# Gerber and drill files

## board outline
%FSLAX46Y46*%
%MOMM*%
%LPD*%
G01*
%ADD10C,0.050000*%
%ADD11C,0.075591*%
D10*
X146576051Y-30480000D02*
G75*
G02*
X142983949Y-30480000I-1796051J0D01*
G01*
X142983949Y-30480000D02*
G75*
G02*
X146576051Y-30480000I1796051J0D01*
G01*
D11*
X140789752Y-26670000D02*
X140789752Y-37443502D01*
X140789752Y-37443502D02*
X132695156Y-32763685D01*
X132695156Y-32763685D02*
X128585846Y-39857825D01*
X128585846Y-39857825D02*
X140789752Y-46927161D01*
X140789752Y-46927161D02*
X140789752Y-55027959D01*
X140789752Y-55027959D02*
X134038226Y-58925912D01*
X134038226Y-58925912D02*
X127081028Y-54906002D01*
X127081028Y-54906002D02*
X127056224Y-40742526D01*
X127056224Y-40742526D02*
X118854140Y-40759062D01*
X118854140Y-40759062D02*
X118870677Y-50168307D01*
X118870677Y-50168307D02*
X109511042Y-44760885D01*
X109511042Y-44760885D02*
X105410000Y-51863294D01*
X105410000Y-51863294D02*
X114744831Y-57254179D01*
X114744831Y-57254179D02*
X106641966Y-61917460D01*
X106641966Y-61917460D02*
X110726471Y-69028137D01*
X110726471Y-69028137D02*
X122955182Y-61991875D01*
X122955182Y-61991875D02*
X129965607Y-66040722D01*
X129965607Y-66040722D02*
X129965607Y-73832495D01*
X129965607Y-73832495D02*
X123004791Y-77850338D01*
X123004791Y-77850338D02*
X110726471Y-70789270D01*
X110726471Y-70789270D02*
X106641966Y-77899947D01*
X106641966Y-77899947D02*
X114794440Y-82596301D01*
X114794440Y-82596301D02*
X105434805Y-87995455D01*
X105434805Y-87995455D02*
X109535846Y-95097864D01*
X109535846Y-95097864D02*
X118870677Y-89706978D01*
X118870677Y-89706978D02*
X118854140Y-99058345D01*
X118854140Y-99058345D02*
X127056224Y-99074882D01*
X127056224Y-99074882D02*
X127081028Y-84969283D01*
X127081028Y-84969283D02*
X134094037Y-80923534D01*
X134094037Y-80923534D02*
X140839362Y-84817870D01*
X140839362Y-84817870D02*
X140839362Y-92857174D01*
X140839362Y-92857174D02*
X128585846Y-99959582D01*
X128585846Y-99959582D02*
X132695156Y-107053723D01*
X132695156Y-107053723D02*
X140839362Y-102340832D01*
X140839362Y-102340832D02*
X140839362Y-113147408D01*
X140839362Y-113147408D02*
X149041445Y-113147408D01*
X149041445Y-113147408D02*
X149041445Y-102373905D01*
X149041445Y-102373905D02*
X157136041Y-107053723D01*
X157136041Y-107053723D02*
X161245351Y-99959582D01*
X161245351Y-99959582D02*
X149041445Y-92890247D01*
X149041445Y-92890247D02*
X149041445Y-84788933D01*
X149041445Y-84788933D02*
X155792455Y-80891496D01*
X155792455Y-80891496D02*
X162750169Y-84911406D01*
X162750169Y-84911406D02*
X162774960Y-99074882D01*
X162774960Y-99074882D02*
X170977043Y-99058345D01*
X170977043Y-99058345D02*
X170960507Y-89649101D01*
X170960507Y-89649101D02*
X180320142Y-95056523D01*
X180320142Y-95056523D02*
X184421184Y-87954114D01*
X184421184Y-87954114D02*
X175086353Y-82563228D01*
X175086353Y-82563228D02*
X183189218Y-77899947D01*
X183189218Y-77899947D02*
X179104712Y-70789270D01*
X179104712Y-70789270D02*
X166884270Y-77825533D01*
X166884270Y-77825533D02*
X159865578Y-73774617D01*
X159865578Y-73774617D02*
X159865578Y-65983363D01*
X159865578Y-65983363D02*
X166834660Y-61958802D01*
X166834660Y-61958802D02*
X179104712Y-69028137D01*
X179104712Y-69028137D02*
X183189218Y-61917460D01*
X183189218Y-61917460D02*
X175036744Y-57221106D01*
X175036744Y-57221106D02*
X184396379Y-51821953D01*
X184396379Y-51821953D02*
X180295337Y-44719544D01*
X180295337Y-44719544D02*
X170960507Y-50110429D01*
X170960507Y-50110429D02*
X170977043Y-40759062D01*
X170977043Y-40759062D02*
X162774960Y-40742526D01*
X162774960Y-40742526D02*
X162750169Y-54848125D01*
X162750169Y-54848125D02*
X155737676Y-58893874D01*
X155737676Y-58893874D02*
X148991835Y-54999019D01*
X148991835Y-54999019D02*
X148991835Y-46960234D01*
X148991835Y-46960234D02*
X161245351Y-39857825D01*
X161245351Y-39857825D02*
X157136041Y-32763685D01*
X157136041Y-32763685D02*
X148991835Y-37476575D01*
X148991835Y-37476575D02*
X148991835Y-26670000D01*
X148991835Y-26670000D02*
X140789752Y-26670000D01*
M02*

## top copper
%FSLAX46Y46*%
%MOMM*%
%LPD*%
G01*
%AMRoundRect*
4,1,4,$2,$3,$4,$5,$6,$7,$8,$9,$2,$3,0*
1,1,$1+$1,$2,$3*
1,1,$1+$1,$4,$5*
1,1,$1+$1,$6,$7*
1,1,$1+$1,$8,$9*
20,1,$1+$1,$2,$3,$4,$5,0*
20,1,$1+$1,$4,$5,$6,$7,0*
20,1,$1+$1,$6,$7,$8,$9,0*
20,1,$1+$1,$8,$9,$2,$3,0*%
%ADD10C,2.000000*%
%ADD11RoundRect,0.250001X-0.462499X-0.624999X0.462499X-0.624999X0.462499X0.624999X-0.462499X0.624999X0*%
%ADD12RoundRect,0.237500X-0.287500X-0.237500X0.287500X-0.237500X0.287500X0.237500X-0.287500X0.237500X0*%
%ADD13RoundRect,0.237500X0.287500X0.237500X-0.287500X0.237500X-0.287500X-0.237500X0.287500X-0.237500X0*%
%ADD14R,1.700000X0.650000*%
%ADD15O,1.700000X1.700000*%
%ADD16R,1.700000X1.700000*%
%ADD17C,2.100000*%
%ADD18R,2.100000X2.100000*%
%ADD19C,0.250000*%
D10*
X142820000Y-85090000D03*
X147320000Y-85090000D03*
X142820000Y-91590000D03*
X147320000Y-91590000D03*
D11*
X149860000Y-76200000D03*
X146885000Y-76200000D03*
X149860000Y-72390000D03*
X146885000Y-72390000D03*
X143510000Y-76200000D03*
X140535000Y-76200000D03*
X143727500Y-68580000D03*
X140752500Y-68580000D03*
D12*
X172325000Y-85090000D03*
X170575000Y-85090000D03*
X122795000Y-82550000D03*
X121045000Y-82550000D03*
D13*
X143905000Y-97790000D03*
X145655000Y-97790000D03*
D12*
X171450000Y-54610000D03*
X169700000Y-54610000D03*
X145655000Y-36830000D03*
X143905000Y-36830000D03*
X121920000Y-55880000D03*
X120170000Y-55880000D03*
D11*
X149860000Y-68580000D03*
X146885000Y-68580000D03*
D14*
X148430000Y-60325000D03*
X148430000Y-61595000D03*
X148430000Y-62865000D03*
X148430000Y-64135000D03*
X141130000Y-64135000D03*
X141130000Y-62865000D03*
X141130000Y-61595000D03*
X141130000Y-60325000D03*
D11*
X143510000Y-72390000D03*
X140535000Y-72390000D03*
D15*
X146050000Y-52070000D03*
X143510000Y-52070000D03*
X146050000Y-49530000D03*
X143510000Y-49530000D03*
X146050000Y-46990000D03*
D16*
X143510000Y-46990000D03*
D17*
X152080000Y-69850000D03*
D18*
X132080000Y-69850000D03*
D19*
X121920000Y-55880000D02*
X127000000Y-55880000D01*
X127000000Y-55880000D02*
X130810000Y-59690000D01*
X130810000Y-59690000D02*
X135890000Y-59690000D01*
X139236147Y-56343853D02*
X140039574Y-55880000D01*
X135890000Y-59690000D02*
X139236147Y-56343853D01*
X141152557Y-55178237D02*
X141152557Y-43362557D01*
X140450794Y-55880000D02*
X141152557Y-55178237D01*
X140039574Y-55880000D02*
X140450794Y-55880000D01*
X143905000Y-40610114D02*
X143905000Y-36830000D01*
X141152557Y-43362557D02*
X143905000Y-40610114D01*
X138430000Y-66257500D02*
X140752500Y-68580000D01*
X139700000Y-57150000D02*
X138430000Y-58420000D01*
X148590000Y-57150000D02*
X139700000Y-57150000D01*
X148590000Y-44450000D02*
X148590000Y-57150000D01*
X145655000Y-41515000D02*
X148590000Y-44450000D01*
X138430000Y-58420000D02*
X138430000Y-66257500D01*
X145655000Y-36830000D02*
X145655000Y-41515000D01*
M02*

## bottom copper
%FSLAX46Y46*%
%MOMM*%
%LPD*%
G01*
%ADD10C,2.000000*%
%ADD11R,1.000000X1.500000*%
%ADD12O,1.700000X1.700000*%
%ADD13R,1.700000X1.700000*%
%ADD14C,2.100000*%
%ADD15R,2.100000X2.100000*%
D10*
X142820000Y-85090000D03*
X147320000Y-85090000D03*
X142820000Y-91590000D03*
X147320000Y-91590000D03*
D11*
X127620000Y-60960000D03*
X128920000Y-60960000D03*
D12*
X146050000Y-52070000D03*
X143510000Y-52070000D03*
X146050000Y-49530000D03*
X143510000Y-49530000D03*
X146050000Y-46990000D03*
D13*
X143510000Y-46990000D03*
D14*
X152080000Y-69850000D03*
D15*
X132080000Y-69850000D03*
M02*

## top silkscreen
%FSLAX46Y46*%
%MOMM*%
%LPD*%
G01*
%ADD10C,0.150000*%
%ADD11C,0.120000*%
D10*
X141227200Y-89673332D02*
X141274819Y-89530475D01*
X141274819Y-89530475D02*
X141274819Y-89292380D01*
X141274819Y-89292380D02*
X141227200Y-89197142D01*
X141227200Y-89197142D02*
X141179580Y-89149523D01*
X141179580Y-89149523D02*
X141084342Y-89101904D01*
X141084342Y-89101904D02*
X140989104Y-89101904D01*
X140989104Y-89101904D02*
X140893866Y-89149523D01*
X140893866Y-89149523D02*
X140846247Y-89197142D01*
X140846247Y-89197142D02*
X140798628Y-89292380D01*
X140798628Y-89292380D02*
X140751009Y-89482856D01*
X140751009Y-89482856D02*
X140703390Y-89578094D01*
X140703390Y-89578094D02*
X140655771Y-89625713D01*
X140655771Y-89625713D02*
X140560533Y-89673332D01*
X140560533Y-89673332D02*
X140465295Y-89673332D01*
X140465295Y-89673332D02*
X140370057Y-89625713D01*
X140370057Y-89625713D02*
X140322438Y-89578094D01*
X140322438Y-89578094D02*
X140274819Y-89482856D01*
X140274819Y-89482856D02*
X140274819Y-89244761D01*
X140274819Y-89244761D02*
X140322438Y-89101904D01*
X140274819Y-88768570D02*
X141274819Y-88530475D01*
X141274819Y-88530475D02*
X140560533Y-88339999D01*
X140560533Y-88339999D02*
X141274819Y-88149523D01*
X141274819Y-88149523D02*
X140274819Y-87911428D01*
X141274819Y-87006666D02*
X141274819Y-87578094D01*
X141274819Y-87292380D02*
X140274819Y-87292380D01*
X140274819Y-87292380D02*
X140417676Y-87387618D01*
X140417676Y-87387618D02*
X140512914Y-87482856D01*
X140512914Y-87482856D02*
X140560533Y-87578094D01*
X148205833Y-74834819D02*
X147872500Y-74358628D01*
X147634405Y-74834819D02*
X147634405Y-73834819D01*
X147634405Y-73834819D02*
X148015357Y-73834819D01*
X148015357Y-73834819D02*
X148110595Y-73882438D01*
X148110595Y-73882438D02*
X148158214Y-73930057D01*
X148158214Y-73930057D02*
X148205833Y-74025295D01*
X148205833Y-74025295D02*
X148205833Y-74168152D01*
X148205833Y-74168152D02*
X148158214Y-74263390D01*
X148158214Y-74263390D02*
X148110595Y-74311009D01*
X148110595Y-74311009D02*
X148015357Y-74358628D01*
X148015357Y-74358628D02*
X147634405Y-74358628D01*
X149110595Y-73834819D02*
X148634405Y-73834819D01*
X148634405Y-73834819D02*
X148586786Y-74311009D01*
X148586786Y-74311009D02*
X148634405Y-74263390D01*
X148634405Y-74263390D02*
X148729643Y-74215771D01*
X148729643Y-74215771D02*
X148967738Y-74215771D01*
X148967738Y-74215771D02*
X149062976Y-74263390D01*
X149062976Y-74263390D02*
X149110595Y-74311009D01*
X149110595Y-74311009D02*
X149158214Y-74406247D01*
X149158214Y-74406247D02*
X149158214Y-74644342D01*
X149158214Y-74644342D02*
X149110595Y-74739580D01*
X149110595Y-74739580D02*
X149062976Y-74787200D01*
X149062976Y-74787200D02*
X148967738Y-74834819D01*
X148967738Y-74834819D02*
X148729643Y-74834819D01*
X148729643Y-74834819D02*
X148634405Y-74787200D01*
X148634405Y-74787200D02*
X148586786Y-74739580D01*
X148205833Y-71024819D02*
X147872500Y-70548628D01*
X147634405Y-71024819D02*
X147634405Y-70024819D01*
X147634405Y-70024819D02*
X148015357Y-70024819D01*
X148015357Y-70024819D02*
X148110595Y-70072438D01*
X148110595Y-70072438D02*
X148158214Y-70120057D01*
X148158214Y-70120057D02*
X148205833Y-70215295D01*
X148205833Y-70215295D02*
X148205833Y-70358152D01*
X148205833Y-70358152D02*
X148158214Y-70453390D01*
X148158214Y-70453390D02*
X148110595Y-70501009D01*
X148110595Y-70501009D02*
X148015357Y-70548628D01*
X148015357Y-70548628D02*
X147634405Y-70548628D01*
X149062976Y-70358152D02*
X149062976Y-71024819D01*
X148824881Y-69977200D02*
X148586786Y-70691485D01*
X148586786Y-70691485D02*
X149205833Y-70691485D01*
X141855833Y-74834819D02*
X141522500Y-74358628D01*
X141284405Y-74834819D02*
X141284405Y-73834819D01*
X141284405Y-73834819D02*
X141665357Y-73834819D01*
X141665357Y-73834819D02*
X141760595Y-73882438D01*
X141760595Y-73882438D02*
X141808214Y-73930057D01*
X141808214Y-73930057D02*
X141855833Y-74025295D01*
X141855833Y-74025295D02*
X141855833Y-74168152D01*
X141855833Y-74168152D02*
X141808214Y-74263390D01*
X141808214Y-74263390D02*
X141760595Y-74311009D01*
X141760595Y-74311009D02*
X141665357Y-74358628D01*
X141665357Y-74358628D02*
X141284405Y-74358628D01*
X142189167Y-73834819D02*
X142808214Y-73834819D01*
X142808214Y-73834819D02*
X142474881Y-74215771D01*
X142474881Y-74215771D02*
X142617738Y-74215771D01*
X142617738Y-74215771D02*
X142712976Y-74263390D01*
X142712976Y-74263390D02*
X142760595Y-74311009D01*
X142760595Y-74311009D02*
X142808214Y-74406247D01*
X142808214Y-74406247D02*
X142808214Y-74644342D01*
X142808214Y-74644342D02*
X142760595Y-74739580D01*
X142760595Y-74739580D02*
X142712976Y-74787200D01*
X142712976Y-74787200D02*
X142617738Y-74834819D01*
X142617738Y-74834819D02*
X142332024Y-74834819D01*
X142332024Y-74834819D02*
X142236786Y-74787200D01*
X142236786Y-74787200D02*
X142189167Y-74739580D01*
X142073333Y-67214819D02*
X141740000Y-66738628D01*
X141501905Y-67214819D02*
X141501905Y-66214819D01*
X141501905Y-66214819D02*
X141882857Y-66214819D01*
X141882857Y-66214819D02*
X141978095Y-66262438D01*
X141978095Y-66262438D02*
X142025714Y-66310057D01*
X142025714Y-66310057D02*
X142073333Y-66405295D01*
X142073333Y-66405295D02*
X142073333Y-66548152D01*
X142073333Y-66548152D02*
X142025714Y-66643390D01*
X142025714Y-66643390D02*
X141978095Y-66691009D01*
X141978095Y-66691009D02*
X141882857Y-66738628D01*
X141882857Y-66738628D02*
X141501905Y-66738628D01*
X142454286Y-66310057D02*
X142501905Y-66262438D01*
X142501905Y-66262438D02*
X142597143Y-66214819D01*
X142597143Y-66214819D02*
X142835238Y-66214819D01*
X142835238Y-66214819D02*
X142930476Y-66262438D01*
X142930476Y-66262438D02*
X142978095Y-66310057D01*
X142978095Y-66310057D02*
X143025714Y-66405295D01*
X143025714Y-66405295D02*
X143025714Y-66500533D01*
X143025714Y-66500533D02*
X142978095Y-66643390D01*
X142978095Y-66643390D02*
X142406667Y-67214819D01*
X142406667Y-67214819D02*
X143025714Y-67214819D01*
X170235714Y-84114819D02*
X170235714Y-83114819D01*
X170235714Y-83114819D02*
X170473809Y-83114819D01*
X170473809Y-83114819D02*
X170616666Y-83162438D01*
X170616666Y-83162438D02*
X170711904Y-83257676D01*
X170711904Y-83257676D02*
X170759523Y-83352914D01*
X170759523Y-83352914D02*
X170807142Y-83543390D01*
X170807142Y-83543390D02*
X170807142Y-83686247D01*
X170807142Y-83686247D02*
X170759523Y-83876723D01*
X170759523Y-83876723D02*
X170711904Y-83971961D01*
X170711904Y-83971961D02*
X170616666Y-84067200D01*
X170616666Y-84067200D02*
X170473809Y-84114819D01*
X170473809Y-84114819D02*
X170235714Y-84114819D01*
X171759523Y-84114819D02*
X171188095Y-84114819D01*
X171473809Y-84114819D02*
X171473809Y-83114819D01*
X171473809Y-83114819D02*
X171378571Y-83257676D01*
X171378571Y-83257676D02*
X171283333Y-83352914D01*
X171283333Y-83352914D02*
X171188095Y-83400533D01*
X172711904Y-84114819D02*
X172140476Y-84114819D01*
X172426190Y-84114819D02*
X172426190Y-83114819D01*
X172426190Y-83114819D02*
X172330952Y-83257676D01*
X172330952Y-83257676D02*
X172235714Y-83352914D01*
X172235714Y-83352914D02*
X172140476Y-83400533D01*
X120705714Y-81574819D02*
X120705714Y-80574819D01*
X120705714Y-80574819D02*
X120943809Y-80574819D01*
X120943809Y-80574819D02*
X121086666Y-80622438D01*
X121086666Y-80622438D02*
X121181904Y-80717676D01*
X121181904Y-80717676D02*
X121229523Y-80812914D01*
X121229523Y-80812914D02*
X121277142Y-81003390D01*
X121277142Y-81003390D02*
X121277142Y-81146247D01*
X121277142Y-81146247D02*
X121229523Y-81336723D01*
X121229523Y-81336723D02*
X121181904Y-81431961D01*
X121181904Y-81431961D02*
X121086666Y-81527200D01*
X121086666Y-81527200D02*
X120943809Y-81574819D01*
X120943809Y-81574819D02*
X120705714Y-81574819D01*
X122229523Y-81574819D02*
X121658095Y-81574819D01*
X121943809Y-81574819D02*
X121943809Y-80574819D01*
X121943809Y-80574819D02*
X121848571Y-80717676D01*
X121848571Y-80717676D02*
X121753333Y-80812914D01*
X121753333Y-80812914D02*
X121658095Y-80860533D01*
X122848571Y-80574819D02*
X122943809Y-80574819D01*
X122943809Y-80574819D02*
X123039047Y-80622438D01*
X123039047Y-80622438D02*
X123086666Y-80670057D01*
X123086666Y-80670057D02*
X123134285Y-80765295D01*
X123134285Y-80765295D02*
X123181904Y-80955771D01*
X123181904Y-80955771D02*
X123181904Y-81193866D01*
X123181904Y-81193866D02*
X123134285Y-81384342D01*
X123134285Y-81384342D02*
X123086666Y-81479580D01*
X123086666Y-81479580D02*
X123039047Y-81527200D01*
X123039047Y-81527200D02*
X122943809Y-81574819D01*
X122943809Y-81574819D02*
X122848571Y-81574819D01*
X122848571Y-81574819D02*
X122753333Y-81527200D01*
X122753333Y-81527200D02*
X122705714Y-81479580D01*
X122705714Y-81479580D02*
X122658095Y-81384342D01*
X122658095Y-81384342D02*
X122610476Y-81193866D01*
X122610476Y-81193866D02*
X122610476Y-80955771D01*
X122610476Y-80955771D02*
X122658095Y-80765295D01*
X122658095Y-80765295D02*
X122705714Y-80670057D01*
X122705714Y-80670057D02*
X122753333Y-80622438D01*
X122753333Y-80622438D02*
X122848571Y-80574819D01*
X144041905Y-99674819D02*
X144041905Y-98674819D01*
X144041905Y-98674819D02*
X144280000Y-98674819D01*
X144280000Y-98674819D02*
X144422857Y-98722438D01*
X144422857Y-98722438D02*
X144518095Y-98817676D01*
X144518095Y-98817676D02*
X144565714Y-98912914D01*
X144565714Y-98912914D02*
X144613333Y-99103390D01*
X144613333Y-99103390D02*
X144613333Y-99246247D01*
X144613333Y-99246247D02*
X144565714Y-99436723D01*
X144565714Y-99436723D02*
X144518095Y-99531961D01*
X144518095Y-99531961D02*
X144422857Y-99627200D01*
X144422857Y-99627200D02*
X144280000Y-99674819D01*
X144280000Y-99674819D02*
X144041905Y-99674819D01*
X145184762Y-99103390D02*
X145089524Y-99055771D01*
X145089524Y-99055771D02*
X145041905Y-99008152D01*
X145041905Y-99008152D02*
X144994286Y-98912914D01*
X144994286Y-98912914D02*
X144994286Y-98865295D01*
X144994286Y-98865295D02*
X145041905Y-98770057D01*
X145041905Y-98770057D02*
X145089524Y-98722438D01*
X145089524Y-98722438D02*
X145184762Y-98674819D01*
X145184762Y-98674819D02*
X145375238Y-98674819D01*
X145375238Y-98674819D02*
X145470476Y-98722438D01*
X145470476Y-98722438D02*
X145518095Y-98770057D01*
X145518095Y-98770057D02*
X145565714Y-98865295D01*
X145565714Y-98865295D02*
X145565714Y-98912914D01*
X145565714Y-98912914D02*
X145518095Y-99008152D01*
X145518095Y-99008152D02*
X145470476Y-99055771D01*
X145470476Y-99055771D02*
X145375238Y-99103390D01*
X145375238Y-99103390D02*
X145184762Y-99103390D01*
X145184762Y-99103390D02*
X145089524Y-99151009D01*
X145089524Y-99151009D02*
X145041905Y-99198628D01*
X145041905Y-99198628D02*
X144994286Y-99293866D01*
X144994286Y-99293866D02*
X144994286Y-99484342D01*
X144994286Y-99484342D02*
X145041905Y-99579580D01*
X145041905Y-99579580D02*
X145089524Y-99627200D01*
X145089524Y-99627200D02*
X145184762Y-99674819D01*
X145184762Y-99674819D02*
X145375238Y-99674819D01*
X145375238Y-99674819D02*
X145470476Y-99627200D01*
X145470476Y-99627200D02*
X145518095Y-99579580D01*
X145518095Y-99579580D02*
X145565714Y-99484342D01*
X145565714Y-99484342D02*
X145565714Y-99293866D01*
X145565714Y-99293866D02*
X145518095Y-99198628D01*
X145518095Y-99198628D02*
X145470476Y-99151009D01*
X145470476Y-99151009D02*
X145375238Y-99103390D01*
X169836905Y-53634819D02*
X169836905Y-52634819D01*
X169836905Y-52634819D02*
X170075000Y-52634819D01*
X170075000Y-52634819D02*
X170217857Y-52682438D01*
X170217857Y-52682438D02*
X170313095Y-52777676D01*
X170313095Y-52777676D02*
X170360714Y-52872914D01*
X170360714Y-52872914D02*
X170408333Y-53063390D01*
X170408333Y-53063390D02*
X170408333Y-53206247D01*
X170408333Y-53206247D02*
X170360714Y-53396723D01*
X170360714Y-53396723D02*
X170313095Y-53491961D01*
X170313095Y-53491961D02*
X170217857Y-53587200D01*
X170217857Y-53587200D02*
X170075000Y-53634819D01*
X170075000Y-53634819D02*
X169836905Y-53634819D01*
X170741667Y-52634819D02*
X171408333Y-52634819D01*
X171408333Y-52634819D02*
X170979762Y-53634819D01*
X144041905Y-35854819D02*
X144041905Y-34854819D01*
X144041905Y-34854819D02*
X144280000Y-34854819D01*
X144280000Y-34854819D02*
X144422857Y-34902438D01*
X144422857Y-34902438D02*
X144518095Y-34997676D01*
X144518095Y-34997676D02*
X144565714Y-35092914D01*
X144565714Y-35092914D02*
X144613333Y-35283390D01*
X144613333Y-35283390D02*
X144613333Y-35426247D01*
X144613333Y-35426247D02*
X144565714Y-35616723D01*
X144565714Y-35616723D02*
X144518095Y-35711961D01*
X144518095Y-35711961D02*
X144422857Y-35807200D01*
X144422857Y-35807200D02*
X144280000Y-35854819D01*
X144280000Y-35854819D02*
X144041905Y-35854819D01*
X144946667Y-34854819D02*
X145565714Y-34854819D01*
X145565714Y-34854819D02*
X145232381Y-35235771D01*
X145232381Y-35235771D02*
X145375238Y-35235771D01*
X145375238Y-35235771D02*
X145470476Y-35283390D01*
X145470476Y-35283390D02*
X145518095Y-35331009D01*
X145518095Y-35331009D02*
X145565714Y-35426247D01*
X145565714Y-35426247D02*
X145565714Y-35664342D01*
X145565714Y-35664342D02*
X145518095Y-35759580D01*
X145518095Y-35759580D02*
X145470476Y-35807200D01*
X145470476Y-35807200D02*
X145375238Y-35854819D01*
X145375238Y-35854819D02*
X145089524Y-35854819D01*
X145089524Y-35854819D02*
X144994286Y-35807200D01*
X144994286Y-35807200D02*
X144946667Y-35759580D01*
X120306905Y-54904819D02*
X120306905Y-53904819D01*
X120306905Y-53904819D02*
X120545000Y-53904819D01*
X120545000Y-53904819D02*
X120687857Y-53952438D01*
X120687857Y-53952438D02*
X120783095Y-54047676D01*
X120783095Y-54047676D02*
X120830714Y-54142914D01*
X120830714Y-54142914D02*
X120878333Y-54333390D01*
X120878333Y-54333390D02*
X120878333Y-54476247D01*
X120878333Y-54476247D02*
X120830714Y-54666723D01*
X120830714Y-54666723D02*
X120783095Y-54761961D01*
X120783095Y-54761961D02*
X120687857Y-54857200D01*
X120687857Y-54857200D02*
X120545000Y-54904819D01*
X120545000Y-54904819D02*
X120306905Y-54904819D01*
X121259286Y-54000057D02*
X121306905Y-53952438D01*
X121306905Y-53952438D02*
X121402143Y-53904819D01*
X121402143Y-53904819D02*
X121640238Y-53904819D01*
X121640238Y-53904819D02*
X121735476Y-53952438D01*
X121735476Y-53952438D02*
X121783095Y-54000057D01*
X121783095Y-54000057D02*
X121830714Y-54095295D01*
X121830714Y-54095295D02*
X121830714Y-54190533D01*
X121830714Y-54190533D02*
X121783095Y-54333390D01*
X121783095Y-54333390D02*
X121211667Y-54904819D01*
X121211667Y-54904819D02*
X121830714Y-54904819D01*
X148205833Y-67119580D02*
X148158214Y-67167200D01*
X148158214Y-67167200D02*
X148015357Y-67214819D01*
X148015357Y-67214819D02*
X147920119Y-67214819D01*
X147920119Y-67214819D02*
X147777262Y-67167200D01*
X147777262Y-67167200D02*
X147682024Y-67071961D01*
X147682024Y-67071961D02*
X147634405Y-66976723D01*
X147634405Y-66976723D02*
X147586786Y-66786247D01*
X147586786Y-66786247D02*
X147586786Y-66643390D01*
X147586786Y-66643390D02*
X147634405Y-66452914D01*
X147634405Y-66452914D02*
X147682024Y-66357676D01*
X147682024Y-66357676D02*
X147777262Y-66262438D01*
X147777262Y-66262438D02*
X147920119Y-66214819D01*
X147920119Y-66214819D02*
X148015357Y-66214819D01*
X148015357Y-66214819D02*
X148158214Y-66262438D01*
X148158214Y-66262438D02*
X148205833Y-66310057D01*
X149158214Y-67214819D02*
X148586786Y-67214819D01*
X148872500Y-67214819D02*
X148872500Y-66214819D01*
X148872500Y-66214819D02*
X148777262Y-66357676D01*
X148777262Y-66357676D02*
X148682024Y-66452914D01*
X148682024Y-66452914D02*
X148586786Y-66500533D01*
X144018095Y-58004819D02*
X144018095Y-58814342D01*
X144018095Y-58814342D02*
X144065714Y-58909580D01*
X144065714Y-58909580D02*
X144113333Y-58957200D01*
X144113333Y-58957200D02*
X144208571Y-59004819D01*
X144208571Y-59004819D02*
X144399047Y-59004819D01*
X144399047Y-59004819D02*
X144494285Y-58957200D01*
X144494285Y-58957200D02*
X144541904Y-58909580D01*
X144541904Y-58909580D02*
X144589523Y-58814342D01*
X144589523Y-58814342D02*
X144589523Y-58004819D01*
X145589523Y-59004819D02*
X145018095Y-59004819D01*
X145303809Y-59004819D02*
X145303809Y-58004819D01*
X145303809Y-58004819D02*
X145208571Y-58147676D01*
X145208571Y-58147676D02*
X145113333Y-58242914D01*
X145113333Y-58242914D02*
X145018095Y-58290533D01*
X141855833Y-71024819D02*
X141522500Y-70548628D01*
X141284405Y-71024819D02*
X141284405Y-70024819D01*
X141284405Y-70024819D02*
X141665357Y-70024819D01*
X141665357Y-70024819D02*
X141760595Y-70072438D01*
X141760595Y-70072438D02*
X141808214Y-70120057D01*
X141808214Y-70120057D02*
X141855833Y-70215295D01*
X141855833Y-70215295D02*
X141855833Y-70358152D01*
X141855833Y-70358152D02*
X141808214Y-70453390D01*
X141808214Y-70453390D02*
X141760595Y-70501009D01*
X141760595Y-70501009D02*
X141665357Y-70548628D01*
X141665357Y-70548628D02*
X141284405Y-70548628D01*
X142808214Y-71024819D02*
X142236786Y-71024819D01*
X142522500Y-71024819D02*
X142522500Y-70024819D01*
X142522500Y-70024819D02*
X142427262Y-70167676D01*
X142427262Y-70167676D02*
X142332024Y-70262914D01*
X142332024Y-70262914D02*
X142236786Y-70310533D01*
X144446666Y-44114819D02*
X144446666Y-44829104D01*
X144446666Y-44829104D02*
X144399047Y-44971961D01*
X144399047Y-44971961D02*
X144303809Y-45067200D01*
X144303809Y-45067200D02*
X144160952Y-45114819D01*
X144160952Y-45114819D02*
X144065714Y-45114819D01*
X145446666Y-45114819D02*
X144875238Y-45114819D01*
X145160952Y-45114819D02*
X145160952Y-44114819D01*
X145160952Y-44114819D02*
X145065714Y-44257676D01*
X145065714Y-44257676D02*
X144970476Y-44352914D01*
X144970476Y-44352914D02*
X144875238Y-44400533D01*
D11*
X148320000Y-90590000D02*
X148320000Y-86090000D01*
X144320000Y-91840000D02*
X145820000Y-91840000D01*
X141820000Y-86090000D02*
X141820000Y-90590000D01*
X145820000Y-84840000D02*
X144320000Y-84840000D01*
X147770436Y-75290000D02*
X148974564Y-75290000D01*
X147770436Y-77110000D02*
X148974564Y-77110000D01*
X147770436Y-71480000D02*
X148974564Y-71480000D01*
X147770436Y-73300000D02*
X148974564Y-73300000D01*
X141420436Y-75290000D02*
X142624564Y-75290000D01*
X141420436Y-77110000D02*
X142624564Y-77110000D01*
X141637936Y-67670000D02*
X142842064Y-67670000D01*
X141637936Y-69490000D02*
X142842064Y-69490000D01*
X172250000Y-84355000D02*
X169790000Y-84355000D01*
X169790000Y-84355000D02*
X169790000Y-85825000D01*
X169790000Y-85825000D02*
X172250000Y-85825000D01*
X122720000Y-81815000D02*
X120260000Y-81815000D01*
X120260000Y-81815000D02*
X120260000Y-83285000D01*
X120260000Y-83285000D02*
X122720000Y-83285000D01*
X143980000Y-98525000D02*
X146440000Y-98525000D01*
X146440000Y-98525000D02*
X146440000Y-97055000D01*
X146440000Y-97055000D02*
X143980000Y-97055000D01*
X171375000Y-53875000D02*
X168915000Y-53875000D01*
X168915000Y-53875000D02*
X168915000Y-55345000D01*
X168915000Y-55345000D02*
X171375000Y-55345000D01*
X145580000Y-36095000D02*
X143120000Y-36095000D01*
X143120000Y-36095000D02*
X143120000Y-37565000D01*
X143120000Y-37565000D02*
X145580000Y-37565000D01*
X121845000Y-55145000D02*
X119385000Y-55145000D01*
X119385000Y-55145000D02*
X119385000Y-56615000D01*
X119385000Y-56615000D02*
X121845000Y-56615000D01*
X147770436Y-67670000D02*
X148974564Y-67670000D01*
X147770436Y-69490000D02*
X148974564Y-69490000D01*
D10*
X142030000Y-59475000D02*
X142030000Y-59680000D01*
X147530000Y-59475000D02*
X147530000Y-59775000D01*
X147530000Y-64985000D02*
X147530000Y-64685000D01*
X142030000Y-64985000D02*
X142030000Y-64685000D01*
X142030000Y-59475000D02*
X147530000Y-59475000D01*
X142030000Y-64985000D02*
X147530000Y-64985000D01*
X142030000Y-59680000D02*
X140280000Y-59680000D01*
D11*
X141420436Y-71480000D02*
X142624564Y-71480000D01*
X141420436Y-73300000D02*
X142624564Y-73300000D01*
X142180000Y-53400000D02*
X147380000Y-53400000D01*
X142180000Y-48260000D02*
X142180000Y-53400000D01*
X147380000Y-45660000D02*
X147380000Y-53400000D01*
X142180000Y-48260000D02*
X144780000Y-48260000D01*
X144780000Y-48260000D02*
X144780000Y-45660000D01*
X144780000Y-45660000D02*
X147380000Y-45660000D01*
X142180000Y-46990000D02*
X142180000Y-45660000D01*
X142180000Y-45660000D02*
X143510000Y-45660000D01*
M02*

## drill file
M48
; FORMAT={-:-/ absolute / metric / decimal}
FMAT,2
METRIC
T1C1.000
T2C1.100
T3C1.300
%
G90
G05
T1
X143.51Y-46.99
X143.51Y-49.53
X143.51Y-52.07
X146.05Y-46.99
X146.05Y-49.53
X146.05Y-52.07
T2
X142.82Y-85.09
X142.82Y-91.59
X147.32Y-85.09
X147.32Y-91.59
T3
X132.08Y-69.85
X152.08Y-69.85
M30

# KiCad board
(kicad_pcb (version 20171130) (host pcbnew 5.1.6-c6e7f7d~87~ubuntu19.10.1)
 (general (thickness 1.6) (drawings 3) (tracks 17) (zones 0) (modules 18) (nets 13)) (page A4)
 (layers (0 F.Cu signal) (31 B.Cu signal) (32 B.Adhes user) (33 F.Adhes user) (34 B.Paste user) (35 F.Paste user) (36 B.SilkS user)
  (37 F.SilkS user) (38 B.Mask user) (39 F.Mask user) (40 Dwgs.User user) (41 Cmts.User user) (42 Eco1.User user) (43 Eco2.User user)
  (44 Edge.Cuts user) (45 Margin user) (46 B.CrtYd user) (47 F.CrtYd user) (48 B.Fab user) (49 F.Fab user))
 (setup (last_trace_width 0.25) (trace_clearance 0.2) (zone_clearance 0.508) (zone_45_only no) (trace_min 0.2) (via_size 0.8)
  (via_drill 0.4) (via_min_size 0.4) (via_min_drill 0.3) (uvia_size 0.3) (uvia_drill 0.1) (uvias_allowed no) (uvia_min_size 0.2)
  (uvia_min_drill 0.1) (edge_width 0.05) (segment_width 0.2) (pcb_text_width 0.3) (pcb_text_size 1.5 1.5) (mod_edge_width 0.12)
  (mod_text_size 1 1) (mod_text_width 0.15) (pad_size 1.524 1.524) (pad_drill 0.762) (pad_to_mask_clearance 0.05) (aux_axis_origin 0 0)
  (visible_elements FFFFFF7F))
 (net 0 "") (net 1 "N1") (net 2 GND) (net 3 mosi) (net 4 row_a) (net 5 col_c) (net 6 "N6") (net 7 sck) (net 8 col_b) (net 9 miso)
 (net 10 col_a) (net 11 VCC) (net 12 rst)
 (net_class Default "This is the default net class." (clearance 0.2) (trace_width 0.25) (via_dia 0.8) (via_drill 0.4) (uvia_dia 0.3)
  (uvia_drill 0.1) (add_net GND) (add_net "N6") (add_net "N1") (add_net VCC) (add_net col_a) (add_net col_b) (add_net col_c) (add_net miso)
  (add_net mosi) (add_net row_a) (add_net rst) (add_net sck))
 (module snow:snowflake (layer F.Cu) (at 105.41 26.67)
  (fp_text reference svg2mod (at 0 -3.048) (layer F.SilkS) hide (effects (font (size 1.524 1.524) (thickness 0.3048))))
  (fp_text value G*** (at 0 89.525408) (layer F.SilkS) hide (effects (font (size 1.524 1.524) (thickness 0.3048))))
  (fp_line (start 35.379752 0) (end 35.379752 10.773502) (layer Edge.Cuts) (width 0.075591))
  (fp_line (start 35.379752 10.773502) (end 27.285156 6.093685) (layer Edge.Cuts) (width 0.075591))
  (fp_line (start 27.285156 6.093685) (end 23.175846 13.187825) (layer Edge.Cuts) (width 0.075591))
  (fp_line (start 23.175846 13.187825) (end 35.379752 20.257161) (layer Edge.Cuts) (width 0.075591))
  (fp_line (start 35.379752 20.257161) (end 35.379752 28.357959) (layer Edge.Cuts) (width 0.075591))
  (fp_line (start 35.379752 28.357959) (end 28.628226 32.255912) (layer Edge.Cuts) (width 0.075591))
  (fp_line (start 28.628226 32.255912) (end 21.671028 28.236002) (layer Edge.Cuts) (width 0.075591))
  (fp_line (start 21.671028 28.236002) (end 21.646224 14.072526) (layer Edge.Cuts) (width 0.075591))
  (fp_line (start 21.646224 14.072526) (end 13.44414 14.089062) (layer Edge.Cuts) (width 0.075591))
  (fp_line (start 13.44414 14.089062) (end 13.460677 23.498307) (layer Edge.Cuts) (width 0.075591))
  (fp_line (start 13.460677 23.498307) (end 4.101042 18.090885) (layer Edge.Cuts) (width 0.075591))
  (fp_line (start 4.101042 18.090885) (end 0 25.193294) (layer Edge.Cuts) (width 0.075591))
  (fp_line (start 0 25.193294) (end 9.334831 30.584179) (layer Edge.Cuts) (width 0.075591))
  (fp_line (start 9.334831 30.584179) (end 1.231966 35.24746) (layer Edge.Cuts) (width 0.075591))
  (fp_line (start 1.231966 35.24746) (end 5.316471 42.358137) (layer Edge.Cuts) (width 0.075591))
  (fp_line (start 5.316471 42.358137) (end 17.545182 35.321875) (layer Edge.Cuts) (width 0.075591))
  (fp_line (start 17.545182 35.321875) (end 24.555607 39.370722) (layer Edge.Cuts) (width 0.075591))
  (fp_line (start 24.555607 39.370722) (end 24.555607 47.162495) (layer Edge.Cuts) (width 0.075591))
  (fp_line (start 24.555607 47.162495) (end 17.594791 51.180338) (layer Edge.Cuts) (width 0.075591))
  (fp_line (start 17.594791 51.180338) (end 5.316471 44.11927) (layer Edge.Cuts) (width 0.075591))
  (fp_line (start 5.316471 44.11927) (end 1.231966 51.229947) (layer Edge.Cuts) (width 0.075591))
  (fp_line (start 1.231966 51.229947) (end 9.38444 55.926301) (layer Edge.Cuts) (width 0.075591))
  (fp_line (start 9.38444 55.926301) (end 0.024805 61.325455) (layer Edge.Cuts) (width 0.075591))
  (fp_line (start 0.024805 61.325455) (end 4.125846 68.427864) (layer Edge.Cuts) (width 0.075591))
  (fp_line (start 4.125846 68.427864) (end 13.460677 63.036978) (layer Edge.Cuts) (width 0.075591))
  (fp_line (start 13.460677 63.036978) (end 13.44414 72.388345) (layer Edge.Cuts) (width 0.075591))
  (fp_line (start 13.44414 72.388345) (end 21.646224 72.404882) (layer Edge.Cuts) (width 0.075591))
  (fp_line (start 21.646224 72.404882) (end 21.671028 58.299283) (layer Edge.Cuts) (width 0.075591))
  (fp_line (start 21.671028 58.299283) (end 28.684037 54.253534) (layer Edge.Cuts) (width 0.075591))
  (fp_line (start 28.684037 54.253534) (end 35.429362 58.14787) (layer Edge.Cuts) (width 0.075591))
  (fp_line (start 35.429362 58.14787) (end 35.429362 66.187174) (layer Edge.Cuts) (width 0.075591))
  (fp_line (start 35.429362 66.187174) (end 23.175846 73.289582) (layer Edge.Cuts) (width 0.075591))
  (fp_line (start 23.175846 73.289582) (end 27.285156 80.383723) (layer Edge.Cuts) (width 0.075591))
  (fp_line (start 27.285156 80.383723) (end 35.429362 75.670832) (layer Edge.Cuts) (width 0.075591))
  (fp_line (start 35.429362 75.670832) (end 35.429362 86.477408) (layer Edge.Cuts) (width 0.075591))
  (fp_line (start 35.429362 86.477408) (end 43.631445 86.477408) (layer Edge.Cuts) (width 0.075591))
  (fp_line (start 43.631445 86.477408) (end 43.631445 75.703905) (layer Edge.Cuts) (width 0.075591))
  (fp_line (start 43.631445 75.703905) (end 51.726041 80.383723) (layer Edge.Cuts) (width 0.075591))
  (fp_line (start 51.726041 80.383723) (end 55.835351 73.289582) (layer Edge.Cuts) (width 0.075591))
  (fp_line (start 55.835351 73.289582) (end 43.631445 66.220247) (layer Edge.Cuts) (width 0.075591))
  (fp_line (start 43.631445 66.220247) (end 43.631445 58.118933) (layer Edge.Cuts) (width 0.075591))
  (fp_line (start 43.631445 58.118933) (end 50.382455 54.221496) (layer Edge.Cuts) (width 0.075591))
  (fp_line (start 50.382455 54.221496) (end 57.340169 58.241406) (layer Edge.Cuts) (width 0.075591))
  (fp_line (start 57.340169 58.241406) (end 57.36496 72.404882) (layer Edge.Cuts) (width 0.075591))
  (fp_line (start 57.36496 72.404882) (end 65.567043 72.388345) (layer Edge.Cuts) (width 0.075591))
  (fp_line (start 65.567043 72.388345) (end 65.550507 62.979101) (layer Edge.Cuts) (width 0.075591))
  (fp_line (start 65.550507 62.979101) (end 74.910142 68.386523) (layer Edge.Cuts) (width 0.075591))
  (fp_line (start 74.910142 68.386523) (end 79.011184 61.284114) (layer Edge.Cuts) (width 0.075591))
  (fp_line (start 79.011184 61.284114) (end 69.676353 55.893228) (layer Edge.Cuts) (width 0.075591))
  (fp_line (start 69.676353 55.893228) (end 77.779218 51.229947) (layer Edge.Cuts) (width 0.075591))
  (fp_line (start 77.779218 51.229947) (end 73.694712 44.11927) (layer Edge.Cuts) (width 0.075591))
  (fp_line (start 73.694712 44.11927) (end 61.47427 51.155533) (layer Edge.Cuts) (width 0.075591))
  (fp_line (start 61.47427 51.155533) (end 54.455578 47.104617) (layer Edge.Cuts) (width 0.075591))
  (fp_line (start 54.455578 47.104617) (end 54.455578 39.313363) (layer Edge.Cuts) (width 0.075591))
  (fp_line (start 54.455578 39.313363) (end 61.42466 35.288802) (layer Edge.Cuts) (width 0.075591))
  (fp_line (start 61.42466 35.288802) (end 73.694712 42.358137) (layer Edge.Cuts) (width 0.075591))
  (fp_line (start 73.694712 42.358137) (end 77.779218 35.24746) (layer Edge.Cuts) (width 0.075591))
  (fp_line (start 77.779218 35.24746) (end 69.626744 30.551106) (layer Edge.Cuts) (width 0.075591))
  (fp_line (start 69.626744 30.551106) (end 78.986379 25.151953) (layer Edge.Cuts) (width 0.075591))
  (fp_line (start 78.986379 25.151953) (end 74.885337 18.049544) (layer Edge.Cuts) (width 0.075591))
  (fp_line (start 74.885337 18.049544) (end 65.550507 23.440429) (layer Edge.Cuts) (width 0.075591))
  (fp_line (start 65.550507 23.440429) (end 65.567043 14.089062) (layer Edge.Cuts) (width 0.075591))
  (fp_line (start 65.567043 14.089062) (end 57.36496 14.072526) (layer Edge.Cuts) (width 0.075591))
  (fp_line (start 57.36496 14.072526) (end 57.340169 28.178125) (layer Edge.Cuts) (width 0.075591))
  (fp_line (start 57.340169 28.178125) (end 50.327676 32.223874) (layer Edge.Cuts) (width 0.075591))
  (fp_line (start 50.327676 32.223874) (end 43.581835 28.329019) (layer Edge.Cuts) (width 0.075591))
  (fp_line (start 43.581835 28.329019) (end 43.581835 20.290234) (layer Edge.Cuts) (width 0.075591))
  (fp_line (start 43.581835 20.290234) (end 55.835351 13.187825) (layer Edge.Cuts) (width 0.075591))
  (fp_line (start 55.835351 13.187825) (end 51.726041 6.093685) (layer Edge.Cuts) (width 0.075591))
  (fp_line (start 51.726041 6.093685) (end 43.581835 10.806575) (layer Edge.Cuts) (width 0.075591))
  (fp_line (start 43.581835 10.806575) (end 43.581835 0) (layer Edge.Cuts) (width 0.075591))
  (fp_line (start 43.581835 0) (end 35.379752 0) (layer Edge.Cuts) (width 0.075591)))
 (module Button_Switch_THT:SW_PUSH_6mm (layer F.Cu) (at 142.82 91.59 90)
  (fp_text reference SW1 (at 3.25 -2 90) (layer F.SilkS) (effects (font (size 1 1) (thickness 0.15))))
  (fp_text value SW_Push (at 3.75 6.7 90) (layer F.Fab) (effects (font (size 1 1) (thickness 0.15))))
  (fp_line (start 1 5.5) (end 5.5 5.5) (layer F.SilkS) (width 0.12))
  (fp_line (start -0.25 1.5) (end -0.25 3) (layer F.SilkS) (width 0.12))
  (fp_line (start 5.5 -1) (end 1 -1) (layer F.SilkS) (width 0.12))
  (fp_line (start 6.75 3) (end 6.75 1.5) (layer F.SilkS) (width 0.12))
  (pad 1 thru_hole circle (at 6.5 0 180) (size 2 2) (drill 1.1) (layers *.Cu *.Mask) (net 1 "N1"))
  (pad 2 thru_hole circle (at 6.5 4.5 180) (size 2 2) (drill 1.1) (layers *.Cu *.Mask) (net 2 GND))
  (pad 1 thru_hole circle (at 0 0 180) (size 2 2) (drill 1.1) (layers *.Cu *.Mask) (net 1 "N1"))
  (pad 2 thru_hole circle (at 0 4.5 180) (size 2 2) (drill 1.1) (layers *.Cu *.Mask) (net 2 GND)))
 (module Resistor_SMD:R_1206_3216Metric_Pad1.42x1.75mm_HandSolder (layer F.Cu) (at 148.3725 76.2)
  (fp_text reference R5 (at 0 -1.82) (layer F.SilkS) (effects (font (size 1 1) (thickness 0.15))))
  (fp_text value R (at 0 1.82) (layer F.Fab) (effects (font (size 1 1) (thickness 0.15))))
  (fp_line (start -0.602064 -0.91) (end 0.602064 -0.91) (layer F.SilkS) (width 0.12))
  (fp_line (start -0.602064 0.91) (end 0.602064 0.91) (layer F.SilkS) (width 0.12))
  (pad 2 smd roundrect (at 1.4875 0) (size 1.425 1.75) (layers F.Cu F.Paste F.Mask) (roundrect_rratio 0.175439) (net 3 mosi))
  (pad 1 smd roundrect (at -1.4875 0) (size 1.425 1.75) (layers F.Cu F.Paste F.Mask) (roundrect_rratio 0.175439) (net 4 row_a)))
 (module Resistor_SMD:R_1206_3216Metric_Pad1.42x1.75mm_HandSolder (layer F.Cu) (at 148.3725 72.39)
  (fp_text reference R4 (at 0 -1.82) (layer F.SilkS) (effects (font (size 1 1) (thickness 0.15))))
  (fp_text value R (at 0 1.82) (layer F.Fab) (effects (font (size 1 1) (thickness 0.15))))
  (fp_line (start -0.602064 -0.91) (end 0.602064 -0.91) (layer F.SilkS) (width 0.12))
  (fp_line (start -0.602064 0.91) (end 0.602064 0.91) (layer F.SilkS) (width 0.12))
  (pad 2 smd roundrect (at 1.4875 0) (size 1.425 1.75) (layers F.Cu F.Paste F.Mask) (roundrect_rratio 0.175439) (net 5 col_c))
  (pad 1 smd roundrect (at -1.4875 0) (size 1.425 1.75) (layers F.Cu F.Paste F.Mask) (roundrect_rratio 0.175439) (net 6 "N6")))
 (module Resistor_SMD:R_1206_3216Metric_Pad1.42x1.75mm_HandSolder (layer F.Cu) (at 142.0225 76.2)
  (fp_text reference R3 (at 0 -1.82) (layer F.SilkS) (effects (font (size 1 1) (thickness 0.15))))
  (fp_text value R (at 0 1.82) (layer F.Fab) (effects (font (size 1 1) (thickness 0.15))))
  (fp_line (start -0.602064 -0.91) (end 0.602064 -0.91) (layer F.SilkS) (width 0.12))
  (fp_line (start -0.602064 0.91) (end 0.602064 0.91) (layer F.SilkS) (width 0.12))
  (pad 2 smd roundrect (at 1.4875 0) (size 1.425 1.75) (layers F.Cu F.Paste F.Mask) (roundrect_rratio 0.175439) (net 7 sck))
  (pad 1 smd roundrect (at -1.4875 0) (size 1.425 1.75) (layers F.Cu F.Paste F.Mask) (roundrect_rratio 0.175439) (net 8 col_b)))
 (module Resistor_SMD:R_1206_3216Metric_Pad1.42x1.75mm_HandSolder (layer F.Cu) (at 142.24 68.58)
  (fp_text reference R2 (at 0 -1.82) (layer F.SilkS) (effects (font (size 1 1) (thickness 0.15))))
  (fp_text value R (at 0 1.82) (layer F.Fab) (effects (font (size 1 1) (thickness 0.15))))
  (fp_line (start -0.602064 -0.91) (end 0.602064 -0.91) (layer F.SilkS) (width 0.12))
  (fp_line (start -0.602064 0.91) (end 0.602064 0.91) (layer F.SilkS) (width 0.12))
  (pad 2 smd roundrect (at 1.4875 0) (size 1.425 1.75) (layers F.Cu F.Paste F.Mask) (roundrect_rratio 0.175439) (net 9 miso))
  (pad 1 smd roundrect (at -1.4875 0) (size 1.425 1.75) (layers F.Cu F.Paste F.Mask) (roundrect_rratio 0.175439) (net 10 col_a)))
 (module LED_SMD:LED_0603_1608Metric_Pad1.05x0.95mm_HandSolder (layer F.Cu) (at 171.45 85.09)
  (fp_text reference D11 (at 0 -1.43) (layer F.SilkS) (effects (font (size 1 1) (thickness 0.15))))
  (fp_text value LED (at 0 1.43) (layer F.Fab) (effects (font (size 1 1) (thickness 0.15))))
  (fp_line (start 0.8 -0.735) (end -1.66 -0.735) (layer F.SilkS) (width 0.12))
  (fp_line (start -1.66 -0.735) (end -1.66 0.735) (layer F.SilkS) (width 0.12))
  (fp_line (start -1.66 0.735) (end 0.8 0.735) (layer F.SilkS) (width 0.12))
  (pad 2 smd roundrect (at 0.875 0) (size 1.05 0.95) (layers F.Cu F.Paste F.Mask) (roundrect_rratio 0.25) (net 5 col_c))
  (pad 1 smd roundrect (at -0.875 0) (size 1.05 0.95) (layers F.Cu F.Paste F.Mask) (roundrect_rratio 0.25) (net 4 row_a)))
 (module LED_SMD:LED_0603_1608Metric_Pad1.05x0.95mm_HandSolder (layer F.Cu) (at 121.92 82.55)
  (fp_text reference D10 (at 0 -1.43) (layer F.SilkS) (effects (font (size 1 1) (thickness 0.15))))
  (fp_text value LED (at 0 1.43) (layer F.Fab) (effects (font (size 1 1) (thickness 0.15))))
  (fp_line (start 0.8 -0.735) (end -1.66 -0.735) (layer F.SilkS) (width 0.12))
  (fp_line (start -1.66 -0.735) (end -1.66 0.735) (layer F.SilkS) (width 0.12))
  (fp_line (start -1.66 0.735) (end 0.8 0.735) (layer F.SilkS) (width 0.12))
  (pad 2 smd roundrect (at 0.875 0) (size 1.05 0.95) (layers F.Cu F.Paste F.Mask) (roundrect_rratio 0.25) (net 4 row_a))
  (pad 1 smd roundrect (at -0.875 0) (size 1.05 0.95) (layers F.Cu F.Paste F.Mask) (roundrect_rratio 0.25) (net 5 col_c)))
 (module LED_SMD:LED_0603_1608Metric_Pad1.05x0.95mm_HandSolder (layer F.Cu) (at 144.78 97.79 180)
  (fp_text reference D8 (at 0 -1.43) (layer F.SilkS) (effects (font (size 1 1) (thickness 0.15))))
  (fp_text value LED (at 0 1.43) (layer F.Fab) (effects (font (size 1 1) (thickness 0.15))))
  (fp_line (start 0.8 -0.735) (end -1.66 -0.735) (layer F.SilkS) (width 0.12))
  (fp_line (start -1.66 -0.735) (end -1.66 0.735) (layer F.SilkS) (width 0.12))
  (fp_line (start -1.66 0.735) (end 0.8 0.735) (layer F.SilkS) (width 0.12))
  (pad 2 smd roundrect (at 0.875 0 180) (size 1.05 0.95) (layers F.Cu F.Paste F.Mask) (roundrect_rratio 0.25) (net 8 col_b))
  (pad 1 smd roundrect (at -0.875 0 180) (size 1.05 0.95) (layers F.Cu F.Paste F.Mask) (roundrect_rratio 0.25) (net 4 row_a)))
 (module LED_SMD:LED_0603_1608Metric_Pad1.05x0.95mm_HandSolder (layer F.Cu) (at 170.575 54.61)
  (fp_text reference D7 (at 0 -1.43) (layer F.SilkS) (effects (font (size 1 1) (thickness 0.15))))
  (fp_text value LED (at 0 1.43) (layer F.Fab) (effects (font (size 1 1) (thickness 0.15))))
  (fp_line (start 0.8 -0.735) (end -1.66 -0.735) (layer F.SilkS) (width 0.12))
  (fp_line (start -1.66 -0.735) (end -1.66 0.735) (layer F.SilkS) (width 0.12))
  (fp_line (start -1.66 0.735) (end 0.8 0.735) (layer F.SilkS) (width 0.12))
  (pad 2 smd roundrect (at 0.875 0) (size 1.05 0.95) (layers F.Cu F.Paste F.Mask) (roundrect_rratio 0.25) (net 4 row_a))
  (pad 1 smd roundrect (at -0.875 0) (size 1.05 0.95) (layers F.Cu F.Paste F.Mask) (roundrect_rratio 0.25) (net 8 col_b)))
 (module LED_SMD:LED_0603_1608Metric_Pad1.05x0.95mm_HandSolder (layer F.Cu) (at 144.78 36.83)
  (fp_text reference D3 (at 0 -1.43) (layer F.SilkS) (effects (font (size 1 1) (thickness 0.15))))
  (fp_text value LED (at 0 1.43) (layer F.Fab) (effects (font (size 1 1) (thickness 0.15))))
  (fp_line (start 0.8 -0.735) (end -1.66 -0.735) (layer F.SilkS) (width 0.12))
  (fp_line (start -1.66 -0.735) (end -1.66 0.735) (layer F.SilkS) (width 0.12))
  (fp_line (start -1.66 0.735) (end 0.8 0.735) (layer F.SilkS) (width 0.12))
  (pad 2 smd roundrect (at 0.875 0) (size 1.05 0.95) (layers F.Cu F.Paste F.Mask) (roundrect_rratio 0.25) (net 10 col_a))
  (pad 1 smd roundrect (at -0.875 0) (size 1.05 0.95) (layers F.Cu F.Paste F.Mask) (roundrect_rratio 0.25) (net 4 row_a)))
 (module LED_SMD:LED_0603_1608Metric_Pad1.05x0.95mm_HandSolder (layer F.Cu) (at 121.045 55.88)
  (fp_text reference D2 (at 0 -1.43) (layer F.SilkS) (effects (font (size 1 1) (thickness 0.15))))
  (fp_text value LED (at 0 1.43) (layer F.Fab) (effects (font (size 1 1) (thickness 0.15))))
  (fp_line (start 0.8 -0.735) (end -1.66 -0.735) (layer F.SilkS) (width 0.12))
  (fp_line (start -1.66 -0.735) (end -1.66 0.735) (layer F.SilkS) (width 0.12))
  (fp_line (start -1.66 0.735) (end 0.8 0.735) (layer F.SilkS) (width 0.12))
  (pad 2 smd roundrect (at 0.875 0) (size 1.05 0.95) (layers F.Cu F.Paste F.Mask) (roundrect_rratio 0.25) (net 4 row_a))
  (pad 1 smd roundrect (at -0.875 0) (size 1.05 0.95) (layers F.Cu F.Paste F.Mask) (roundrect_rratio 0.25) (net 10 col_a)))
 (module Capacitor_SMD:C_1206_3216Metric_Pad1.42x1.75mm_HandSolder (layer F.Cu) (at 148.3725 68.58)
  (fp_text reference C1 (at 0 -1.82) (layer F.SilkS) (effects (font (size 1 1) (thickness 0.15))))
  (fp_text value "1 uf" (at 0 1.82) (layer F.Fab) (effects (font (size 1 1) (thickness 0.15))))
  (fp_line (start -0.602064 -0.91) (end 0.602064 -0.91) (layer F.SilkS) (width 0.12))
  (fp_line (start -0.602064 0.91) (end 0.602064 0.91) (layer F.SilkS) (width 0.12))
  (pad 2 smd roundrect (at 1.4875 0) (size 1.425 1.75) (layers F.Cu F.Paste F.Mask) (roundrect_rratio 0.175439) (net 2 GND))
  (pad 1 smd roundrect (at -1.4875 0) (size 1.425 1.75) (layers F.Cu F.Paste F.Mask) (roundrect_rratio 0.175439) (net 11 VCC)))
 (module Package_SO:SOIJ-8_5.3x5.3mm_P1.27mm (layer F.Cu) (at 144.78 62.23)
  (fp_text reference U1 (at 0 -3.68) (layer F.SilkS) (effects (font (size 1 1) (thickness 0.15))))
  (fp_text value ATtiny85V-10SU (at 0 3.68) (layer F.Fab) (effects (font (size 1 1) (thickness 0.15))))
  (fp_line (start -2.75 -2.755) (end -2.75 -2.55) (layer F.SilkS) (width 0.15))
  (fp_line (start 2.75 -2.755) (end 2.75 -2.455) (layer F.SilkS) (width 0.15))
  (fp_line (start 2.75 2.755) (end 2.75 2.455) (layer F.SilkS) (width 0.15))
  (fp_line (start -2.75 2.755) (end -2.75 2.455) (layer F.SilkS) (width 0.15))
  (fp_line (start -2.75 -2.755) (end 2.75 -2.755) (layer F.SilkS) (width 0.15))
  (fp_line (start -2.75 2.755) (end 2.75 2.755) (layer F.SilkS) (width 0.15))
  (fp_line (start -2.75 -2.55) (end -4.5 -2.55) (layer F.SilkS) (width 0.15))
  (pad 8 smd rect (at 3.65 -1.905) (size 1.7 0.65) (layers F.Cu F.Paste F.Mask) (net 11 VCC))
  (pad 7 smd rect (at 3.65 -0.635) (size 1.7 0.65) (layers F.Cu F.Paste F.Mask) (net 7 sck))
  (pad 6 smd rect (at 3.65 0.635) (size 1.7 0.65) (layers F.Cu F.Paste F.Mask) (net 9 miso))
  (pad 5 smd rect (at 3.65 1.905) (size 1.7 0.65) (layers F.Cu F.Paste F.Mask) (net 3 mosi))
  (pad 4 smd rect (at -3.65 1.905) (size 1.7 0.65) (layers F.Cu F.Paste F.Mask) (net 2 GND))
  (pad 3 smd rect (at -3.65 0.635) (size 1.7 0.65) (layers F.Cu F.Paste F.Mask) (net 1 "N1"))
  (pad 2 smd rect (at -3.65 -0.635) (size 1.7 0.65) (layers F.Cu F.Paste F.Mask) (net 6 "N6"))
  (pad 1 smd rect (at -3.65 -1.905) (size 1.7 0.65) (layers F.Cu F.Paste F.Mask) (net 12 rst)))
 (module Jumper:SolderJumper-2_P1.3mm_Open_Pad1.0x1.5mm (layer B.Cu) (at 128.27 60.96)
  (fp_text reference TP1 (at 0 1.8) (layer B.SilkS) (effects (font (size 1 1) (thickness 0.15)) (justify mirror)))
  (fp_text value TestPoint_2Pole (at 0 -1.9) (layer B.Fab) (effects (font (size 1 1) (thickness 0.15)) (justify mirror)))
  (pad 1 smd rect (at -0.65 0) (size 1 1.5) (layers B.Cu B.Mask) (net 12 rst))
  (pad 2 smd rect (at 0.65 0) (size 1 1.5) (layers B.Cu B.Mask) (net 2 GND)))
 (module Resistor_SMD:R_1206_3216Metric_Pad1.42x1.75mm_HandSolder (layer F.Cu) (at 142.0225 72.39)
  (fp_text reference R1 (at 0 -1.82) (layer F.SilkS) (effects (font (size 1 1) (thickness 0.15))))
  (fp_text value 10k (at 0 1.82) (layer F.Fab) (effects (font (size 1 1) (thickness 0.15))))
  (fp_line (start -0.602064 -0.91) (end 0.602064 -0.91) (layer F.SilkS) (width 0.12))
  (fp_line (start -0.602064 0.91) (end 0.602064 0.91) (layer F.SilkS) (width 0.12))
  (pad 2 smd roundrect (at 1.4875 0) (size 1.425 1.75) (layers F.Cu F.Paste F.Mask) (roundrect_rratio 0.175439) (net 12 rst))
  (pad 1 smd roundrect (at -1.4875 0) (size 1.425 1.75) (layers F.Cu F.Paste F.Mask) (roundrect_rratio 0.175439) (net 11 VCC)))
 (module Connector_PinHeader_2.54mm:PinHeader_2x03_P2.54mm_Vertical (layer F.Cu) (at 143.51 46.99)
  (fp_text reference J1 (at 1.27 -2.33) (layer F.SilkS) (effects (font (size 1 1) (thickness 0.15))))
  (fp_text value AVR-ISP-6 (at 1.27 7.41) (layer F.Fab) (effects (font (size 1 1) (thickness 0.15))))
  (fp_line (start -1.33 6.41) (end 3.87 6.41) (layer F.SilkS) (width 0.12))
  (fp_line (start -1.33 1.27) (end -1.33 6.41) (layer F.SilkS) (width 0.12))
  (fp_line (start 3.87 -1.33) (end 3.87 6.41) (layer F.SilkS) (width 0.12))
  (fp_line (start -1.33 1.27) (end 1.27 1.27) (layer F.SilkS) (width 0.12))
  (fp_line (start 1.27 1.27) (end 1.27 -1.33) (layer F.SilkS) (width 0.12))
  (fp_line (start 1.27 -1.33) (end 3.87 -1.33) (layer F.SilkS) (width 0.12))
  (fp_line (start -1.33 0) (end -1.33 -1.33) (layer F.SilkS) (width 0.12))
  (fp_line (start -1.33 -1.33) (end 0 -1.33) (layer F.SilkS) (width 0.12))
  (pad 6 thru_hole oval (at 2.54 5.08) (size 1.7 1.7) (drill 1) (layers *.Cu *.Mask) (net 2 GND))
  (pad 5 thru_hole oval (at 0 5.08) (size 1.7 1.7) (drill 1) (layers *.Cu *.Mask) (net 12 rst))
  (pad 4 thru_hole oval (at 2.54 2.54) (size 1.7 1.7) (drill 1) (layers *.Cu *.Mask) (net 3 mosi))
  (pad 3 thru_hole oval (at 0 2.54) (size 1.7 1.7) (drill 1) (layers *.Cu *.Mask) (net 7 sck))
  (pad 2 thru_hole oval (at 2.54 0) (size 1.7 1.7) (drill 1) (layers *.Cu *.Mask) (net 11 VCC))
  (pad 1 thru_hole rect (at 0 0) (size 1.7 1.7) (drill 1) (layers *.Cu *.Mask) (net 9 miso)))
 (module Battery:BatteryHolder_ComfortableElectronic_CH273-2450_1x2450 (layer B.Cu) (at 132.08 69.85)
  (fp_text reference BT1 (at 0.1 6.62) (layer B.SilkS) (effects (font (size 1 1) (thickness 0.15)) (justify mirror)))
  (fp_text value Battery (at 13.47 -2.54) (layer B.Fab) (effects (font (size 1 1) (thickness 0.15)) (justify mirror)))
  (pad 2 thru_hole circle (at 20 0 90) (size 2.1 2.1) (drill 1.3) (layers *.Cu *.Mask) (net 2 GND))
  (pad 1 thru_hole rect (at 0 0 90) (size 2.1 2.1) (drill 1.3) (layers *.Cu *.Mask) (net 11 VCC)))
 (gr_circle (center 144.78 30.48) (end 146.05 31.75) (layer Edge.Cuts) (width 0.05))
 (segment (start 121.92 55.88) (end 127 55.88) (width 0.25) (layer F.Cu) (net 4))
 (segment (start 127 55.88) (end 130.81 59.69) (width 0.25) (layer F.Cu) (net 4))
 (segment (start 130.81 59.69) (end 135.89 59.69) (width 0.25) (layer F.Cu) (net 4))
 (segment (start 139.236147 56.343853) (end 140.039574 55.88) (width 0.25) (layer F.Cu) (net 4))
 (segment (start 135.89 59.69) (end 139.236147 56.343853) (width 0.25) (layer F.Cu) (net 4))
 (segment (start 141.152557 55.178237) (end 141.152557 43.362557) (width 0.25) (layer F.Cu) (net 4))
 (segment (start 140.450794 55.88) (end 141.152557 55.178237) (width 0.25) (layer F.Cu) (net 4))
 (segment (start 140.039574 55.88) (end 140.450794 55.88) (width 0.25) (layer F.Cu) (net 4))
 (segment (start 143.905 40.610114) (end 143.905 36.83) (width 0.25) (layer F.Cu) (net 4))
 (segment (start 141.152557 43.362557) (end 143.905 40.610114) (width 0.25) (layer F.Cu) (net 4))
 (segment (start 138.43 66.2575) (end 140.7525 68.58) (width 0.25) (layer F.Cu) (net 10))
 (segment (start 139.7 57.15) (end 138.43 58.42) (width 0.25) (layer F.Cu) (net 10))
 (segment (start 148.59 57.15) (end 139.7 57.15) (width 0.25) (layer F.Cu) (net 10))
 (segment (start 148.59 44.45) (end 148.59 57.15) (width 0.25) (layer F.Cu) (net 10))
 (segment (start 145.655 41.515) (end 148.59 44.45) (width 0.25) (layer F.Cu) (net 10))
 (segment (start 138.43 58.42) (end 138.43 66.2575) (width 0.25) (layer F.Cu) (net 10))
 (segment (start 145.655 36.83) (end 145.655 41.515) (width 0.25) (layer F.Cu) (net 10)))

